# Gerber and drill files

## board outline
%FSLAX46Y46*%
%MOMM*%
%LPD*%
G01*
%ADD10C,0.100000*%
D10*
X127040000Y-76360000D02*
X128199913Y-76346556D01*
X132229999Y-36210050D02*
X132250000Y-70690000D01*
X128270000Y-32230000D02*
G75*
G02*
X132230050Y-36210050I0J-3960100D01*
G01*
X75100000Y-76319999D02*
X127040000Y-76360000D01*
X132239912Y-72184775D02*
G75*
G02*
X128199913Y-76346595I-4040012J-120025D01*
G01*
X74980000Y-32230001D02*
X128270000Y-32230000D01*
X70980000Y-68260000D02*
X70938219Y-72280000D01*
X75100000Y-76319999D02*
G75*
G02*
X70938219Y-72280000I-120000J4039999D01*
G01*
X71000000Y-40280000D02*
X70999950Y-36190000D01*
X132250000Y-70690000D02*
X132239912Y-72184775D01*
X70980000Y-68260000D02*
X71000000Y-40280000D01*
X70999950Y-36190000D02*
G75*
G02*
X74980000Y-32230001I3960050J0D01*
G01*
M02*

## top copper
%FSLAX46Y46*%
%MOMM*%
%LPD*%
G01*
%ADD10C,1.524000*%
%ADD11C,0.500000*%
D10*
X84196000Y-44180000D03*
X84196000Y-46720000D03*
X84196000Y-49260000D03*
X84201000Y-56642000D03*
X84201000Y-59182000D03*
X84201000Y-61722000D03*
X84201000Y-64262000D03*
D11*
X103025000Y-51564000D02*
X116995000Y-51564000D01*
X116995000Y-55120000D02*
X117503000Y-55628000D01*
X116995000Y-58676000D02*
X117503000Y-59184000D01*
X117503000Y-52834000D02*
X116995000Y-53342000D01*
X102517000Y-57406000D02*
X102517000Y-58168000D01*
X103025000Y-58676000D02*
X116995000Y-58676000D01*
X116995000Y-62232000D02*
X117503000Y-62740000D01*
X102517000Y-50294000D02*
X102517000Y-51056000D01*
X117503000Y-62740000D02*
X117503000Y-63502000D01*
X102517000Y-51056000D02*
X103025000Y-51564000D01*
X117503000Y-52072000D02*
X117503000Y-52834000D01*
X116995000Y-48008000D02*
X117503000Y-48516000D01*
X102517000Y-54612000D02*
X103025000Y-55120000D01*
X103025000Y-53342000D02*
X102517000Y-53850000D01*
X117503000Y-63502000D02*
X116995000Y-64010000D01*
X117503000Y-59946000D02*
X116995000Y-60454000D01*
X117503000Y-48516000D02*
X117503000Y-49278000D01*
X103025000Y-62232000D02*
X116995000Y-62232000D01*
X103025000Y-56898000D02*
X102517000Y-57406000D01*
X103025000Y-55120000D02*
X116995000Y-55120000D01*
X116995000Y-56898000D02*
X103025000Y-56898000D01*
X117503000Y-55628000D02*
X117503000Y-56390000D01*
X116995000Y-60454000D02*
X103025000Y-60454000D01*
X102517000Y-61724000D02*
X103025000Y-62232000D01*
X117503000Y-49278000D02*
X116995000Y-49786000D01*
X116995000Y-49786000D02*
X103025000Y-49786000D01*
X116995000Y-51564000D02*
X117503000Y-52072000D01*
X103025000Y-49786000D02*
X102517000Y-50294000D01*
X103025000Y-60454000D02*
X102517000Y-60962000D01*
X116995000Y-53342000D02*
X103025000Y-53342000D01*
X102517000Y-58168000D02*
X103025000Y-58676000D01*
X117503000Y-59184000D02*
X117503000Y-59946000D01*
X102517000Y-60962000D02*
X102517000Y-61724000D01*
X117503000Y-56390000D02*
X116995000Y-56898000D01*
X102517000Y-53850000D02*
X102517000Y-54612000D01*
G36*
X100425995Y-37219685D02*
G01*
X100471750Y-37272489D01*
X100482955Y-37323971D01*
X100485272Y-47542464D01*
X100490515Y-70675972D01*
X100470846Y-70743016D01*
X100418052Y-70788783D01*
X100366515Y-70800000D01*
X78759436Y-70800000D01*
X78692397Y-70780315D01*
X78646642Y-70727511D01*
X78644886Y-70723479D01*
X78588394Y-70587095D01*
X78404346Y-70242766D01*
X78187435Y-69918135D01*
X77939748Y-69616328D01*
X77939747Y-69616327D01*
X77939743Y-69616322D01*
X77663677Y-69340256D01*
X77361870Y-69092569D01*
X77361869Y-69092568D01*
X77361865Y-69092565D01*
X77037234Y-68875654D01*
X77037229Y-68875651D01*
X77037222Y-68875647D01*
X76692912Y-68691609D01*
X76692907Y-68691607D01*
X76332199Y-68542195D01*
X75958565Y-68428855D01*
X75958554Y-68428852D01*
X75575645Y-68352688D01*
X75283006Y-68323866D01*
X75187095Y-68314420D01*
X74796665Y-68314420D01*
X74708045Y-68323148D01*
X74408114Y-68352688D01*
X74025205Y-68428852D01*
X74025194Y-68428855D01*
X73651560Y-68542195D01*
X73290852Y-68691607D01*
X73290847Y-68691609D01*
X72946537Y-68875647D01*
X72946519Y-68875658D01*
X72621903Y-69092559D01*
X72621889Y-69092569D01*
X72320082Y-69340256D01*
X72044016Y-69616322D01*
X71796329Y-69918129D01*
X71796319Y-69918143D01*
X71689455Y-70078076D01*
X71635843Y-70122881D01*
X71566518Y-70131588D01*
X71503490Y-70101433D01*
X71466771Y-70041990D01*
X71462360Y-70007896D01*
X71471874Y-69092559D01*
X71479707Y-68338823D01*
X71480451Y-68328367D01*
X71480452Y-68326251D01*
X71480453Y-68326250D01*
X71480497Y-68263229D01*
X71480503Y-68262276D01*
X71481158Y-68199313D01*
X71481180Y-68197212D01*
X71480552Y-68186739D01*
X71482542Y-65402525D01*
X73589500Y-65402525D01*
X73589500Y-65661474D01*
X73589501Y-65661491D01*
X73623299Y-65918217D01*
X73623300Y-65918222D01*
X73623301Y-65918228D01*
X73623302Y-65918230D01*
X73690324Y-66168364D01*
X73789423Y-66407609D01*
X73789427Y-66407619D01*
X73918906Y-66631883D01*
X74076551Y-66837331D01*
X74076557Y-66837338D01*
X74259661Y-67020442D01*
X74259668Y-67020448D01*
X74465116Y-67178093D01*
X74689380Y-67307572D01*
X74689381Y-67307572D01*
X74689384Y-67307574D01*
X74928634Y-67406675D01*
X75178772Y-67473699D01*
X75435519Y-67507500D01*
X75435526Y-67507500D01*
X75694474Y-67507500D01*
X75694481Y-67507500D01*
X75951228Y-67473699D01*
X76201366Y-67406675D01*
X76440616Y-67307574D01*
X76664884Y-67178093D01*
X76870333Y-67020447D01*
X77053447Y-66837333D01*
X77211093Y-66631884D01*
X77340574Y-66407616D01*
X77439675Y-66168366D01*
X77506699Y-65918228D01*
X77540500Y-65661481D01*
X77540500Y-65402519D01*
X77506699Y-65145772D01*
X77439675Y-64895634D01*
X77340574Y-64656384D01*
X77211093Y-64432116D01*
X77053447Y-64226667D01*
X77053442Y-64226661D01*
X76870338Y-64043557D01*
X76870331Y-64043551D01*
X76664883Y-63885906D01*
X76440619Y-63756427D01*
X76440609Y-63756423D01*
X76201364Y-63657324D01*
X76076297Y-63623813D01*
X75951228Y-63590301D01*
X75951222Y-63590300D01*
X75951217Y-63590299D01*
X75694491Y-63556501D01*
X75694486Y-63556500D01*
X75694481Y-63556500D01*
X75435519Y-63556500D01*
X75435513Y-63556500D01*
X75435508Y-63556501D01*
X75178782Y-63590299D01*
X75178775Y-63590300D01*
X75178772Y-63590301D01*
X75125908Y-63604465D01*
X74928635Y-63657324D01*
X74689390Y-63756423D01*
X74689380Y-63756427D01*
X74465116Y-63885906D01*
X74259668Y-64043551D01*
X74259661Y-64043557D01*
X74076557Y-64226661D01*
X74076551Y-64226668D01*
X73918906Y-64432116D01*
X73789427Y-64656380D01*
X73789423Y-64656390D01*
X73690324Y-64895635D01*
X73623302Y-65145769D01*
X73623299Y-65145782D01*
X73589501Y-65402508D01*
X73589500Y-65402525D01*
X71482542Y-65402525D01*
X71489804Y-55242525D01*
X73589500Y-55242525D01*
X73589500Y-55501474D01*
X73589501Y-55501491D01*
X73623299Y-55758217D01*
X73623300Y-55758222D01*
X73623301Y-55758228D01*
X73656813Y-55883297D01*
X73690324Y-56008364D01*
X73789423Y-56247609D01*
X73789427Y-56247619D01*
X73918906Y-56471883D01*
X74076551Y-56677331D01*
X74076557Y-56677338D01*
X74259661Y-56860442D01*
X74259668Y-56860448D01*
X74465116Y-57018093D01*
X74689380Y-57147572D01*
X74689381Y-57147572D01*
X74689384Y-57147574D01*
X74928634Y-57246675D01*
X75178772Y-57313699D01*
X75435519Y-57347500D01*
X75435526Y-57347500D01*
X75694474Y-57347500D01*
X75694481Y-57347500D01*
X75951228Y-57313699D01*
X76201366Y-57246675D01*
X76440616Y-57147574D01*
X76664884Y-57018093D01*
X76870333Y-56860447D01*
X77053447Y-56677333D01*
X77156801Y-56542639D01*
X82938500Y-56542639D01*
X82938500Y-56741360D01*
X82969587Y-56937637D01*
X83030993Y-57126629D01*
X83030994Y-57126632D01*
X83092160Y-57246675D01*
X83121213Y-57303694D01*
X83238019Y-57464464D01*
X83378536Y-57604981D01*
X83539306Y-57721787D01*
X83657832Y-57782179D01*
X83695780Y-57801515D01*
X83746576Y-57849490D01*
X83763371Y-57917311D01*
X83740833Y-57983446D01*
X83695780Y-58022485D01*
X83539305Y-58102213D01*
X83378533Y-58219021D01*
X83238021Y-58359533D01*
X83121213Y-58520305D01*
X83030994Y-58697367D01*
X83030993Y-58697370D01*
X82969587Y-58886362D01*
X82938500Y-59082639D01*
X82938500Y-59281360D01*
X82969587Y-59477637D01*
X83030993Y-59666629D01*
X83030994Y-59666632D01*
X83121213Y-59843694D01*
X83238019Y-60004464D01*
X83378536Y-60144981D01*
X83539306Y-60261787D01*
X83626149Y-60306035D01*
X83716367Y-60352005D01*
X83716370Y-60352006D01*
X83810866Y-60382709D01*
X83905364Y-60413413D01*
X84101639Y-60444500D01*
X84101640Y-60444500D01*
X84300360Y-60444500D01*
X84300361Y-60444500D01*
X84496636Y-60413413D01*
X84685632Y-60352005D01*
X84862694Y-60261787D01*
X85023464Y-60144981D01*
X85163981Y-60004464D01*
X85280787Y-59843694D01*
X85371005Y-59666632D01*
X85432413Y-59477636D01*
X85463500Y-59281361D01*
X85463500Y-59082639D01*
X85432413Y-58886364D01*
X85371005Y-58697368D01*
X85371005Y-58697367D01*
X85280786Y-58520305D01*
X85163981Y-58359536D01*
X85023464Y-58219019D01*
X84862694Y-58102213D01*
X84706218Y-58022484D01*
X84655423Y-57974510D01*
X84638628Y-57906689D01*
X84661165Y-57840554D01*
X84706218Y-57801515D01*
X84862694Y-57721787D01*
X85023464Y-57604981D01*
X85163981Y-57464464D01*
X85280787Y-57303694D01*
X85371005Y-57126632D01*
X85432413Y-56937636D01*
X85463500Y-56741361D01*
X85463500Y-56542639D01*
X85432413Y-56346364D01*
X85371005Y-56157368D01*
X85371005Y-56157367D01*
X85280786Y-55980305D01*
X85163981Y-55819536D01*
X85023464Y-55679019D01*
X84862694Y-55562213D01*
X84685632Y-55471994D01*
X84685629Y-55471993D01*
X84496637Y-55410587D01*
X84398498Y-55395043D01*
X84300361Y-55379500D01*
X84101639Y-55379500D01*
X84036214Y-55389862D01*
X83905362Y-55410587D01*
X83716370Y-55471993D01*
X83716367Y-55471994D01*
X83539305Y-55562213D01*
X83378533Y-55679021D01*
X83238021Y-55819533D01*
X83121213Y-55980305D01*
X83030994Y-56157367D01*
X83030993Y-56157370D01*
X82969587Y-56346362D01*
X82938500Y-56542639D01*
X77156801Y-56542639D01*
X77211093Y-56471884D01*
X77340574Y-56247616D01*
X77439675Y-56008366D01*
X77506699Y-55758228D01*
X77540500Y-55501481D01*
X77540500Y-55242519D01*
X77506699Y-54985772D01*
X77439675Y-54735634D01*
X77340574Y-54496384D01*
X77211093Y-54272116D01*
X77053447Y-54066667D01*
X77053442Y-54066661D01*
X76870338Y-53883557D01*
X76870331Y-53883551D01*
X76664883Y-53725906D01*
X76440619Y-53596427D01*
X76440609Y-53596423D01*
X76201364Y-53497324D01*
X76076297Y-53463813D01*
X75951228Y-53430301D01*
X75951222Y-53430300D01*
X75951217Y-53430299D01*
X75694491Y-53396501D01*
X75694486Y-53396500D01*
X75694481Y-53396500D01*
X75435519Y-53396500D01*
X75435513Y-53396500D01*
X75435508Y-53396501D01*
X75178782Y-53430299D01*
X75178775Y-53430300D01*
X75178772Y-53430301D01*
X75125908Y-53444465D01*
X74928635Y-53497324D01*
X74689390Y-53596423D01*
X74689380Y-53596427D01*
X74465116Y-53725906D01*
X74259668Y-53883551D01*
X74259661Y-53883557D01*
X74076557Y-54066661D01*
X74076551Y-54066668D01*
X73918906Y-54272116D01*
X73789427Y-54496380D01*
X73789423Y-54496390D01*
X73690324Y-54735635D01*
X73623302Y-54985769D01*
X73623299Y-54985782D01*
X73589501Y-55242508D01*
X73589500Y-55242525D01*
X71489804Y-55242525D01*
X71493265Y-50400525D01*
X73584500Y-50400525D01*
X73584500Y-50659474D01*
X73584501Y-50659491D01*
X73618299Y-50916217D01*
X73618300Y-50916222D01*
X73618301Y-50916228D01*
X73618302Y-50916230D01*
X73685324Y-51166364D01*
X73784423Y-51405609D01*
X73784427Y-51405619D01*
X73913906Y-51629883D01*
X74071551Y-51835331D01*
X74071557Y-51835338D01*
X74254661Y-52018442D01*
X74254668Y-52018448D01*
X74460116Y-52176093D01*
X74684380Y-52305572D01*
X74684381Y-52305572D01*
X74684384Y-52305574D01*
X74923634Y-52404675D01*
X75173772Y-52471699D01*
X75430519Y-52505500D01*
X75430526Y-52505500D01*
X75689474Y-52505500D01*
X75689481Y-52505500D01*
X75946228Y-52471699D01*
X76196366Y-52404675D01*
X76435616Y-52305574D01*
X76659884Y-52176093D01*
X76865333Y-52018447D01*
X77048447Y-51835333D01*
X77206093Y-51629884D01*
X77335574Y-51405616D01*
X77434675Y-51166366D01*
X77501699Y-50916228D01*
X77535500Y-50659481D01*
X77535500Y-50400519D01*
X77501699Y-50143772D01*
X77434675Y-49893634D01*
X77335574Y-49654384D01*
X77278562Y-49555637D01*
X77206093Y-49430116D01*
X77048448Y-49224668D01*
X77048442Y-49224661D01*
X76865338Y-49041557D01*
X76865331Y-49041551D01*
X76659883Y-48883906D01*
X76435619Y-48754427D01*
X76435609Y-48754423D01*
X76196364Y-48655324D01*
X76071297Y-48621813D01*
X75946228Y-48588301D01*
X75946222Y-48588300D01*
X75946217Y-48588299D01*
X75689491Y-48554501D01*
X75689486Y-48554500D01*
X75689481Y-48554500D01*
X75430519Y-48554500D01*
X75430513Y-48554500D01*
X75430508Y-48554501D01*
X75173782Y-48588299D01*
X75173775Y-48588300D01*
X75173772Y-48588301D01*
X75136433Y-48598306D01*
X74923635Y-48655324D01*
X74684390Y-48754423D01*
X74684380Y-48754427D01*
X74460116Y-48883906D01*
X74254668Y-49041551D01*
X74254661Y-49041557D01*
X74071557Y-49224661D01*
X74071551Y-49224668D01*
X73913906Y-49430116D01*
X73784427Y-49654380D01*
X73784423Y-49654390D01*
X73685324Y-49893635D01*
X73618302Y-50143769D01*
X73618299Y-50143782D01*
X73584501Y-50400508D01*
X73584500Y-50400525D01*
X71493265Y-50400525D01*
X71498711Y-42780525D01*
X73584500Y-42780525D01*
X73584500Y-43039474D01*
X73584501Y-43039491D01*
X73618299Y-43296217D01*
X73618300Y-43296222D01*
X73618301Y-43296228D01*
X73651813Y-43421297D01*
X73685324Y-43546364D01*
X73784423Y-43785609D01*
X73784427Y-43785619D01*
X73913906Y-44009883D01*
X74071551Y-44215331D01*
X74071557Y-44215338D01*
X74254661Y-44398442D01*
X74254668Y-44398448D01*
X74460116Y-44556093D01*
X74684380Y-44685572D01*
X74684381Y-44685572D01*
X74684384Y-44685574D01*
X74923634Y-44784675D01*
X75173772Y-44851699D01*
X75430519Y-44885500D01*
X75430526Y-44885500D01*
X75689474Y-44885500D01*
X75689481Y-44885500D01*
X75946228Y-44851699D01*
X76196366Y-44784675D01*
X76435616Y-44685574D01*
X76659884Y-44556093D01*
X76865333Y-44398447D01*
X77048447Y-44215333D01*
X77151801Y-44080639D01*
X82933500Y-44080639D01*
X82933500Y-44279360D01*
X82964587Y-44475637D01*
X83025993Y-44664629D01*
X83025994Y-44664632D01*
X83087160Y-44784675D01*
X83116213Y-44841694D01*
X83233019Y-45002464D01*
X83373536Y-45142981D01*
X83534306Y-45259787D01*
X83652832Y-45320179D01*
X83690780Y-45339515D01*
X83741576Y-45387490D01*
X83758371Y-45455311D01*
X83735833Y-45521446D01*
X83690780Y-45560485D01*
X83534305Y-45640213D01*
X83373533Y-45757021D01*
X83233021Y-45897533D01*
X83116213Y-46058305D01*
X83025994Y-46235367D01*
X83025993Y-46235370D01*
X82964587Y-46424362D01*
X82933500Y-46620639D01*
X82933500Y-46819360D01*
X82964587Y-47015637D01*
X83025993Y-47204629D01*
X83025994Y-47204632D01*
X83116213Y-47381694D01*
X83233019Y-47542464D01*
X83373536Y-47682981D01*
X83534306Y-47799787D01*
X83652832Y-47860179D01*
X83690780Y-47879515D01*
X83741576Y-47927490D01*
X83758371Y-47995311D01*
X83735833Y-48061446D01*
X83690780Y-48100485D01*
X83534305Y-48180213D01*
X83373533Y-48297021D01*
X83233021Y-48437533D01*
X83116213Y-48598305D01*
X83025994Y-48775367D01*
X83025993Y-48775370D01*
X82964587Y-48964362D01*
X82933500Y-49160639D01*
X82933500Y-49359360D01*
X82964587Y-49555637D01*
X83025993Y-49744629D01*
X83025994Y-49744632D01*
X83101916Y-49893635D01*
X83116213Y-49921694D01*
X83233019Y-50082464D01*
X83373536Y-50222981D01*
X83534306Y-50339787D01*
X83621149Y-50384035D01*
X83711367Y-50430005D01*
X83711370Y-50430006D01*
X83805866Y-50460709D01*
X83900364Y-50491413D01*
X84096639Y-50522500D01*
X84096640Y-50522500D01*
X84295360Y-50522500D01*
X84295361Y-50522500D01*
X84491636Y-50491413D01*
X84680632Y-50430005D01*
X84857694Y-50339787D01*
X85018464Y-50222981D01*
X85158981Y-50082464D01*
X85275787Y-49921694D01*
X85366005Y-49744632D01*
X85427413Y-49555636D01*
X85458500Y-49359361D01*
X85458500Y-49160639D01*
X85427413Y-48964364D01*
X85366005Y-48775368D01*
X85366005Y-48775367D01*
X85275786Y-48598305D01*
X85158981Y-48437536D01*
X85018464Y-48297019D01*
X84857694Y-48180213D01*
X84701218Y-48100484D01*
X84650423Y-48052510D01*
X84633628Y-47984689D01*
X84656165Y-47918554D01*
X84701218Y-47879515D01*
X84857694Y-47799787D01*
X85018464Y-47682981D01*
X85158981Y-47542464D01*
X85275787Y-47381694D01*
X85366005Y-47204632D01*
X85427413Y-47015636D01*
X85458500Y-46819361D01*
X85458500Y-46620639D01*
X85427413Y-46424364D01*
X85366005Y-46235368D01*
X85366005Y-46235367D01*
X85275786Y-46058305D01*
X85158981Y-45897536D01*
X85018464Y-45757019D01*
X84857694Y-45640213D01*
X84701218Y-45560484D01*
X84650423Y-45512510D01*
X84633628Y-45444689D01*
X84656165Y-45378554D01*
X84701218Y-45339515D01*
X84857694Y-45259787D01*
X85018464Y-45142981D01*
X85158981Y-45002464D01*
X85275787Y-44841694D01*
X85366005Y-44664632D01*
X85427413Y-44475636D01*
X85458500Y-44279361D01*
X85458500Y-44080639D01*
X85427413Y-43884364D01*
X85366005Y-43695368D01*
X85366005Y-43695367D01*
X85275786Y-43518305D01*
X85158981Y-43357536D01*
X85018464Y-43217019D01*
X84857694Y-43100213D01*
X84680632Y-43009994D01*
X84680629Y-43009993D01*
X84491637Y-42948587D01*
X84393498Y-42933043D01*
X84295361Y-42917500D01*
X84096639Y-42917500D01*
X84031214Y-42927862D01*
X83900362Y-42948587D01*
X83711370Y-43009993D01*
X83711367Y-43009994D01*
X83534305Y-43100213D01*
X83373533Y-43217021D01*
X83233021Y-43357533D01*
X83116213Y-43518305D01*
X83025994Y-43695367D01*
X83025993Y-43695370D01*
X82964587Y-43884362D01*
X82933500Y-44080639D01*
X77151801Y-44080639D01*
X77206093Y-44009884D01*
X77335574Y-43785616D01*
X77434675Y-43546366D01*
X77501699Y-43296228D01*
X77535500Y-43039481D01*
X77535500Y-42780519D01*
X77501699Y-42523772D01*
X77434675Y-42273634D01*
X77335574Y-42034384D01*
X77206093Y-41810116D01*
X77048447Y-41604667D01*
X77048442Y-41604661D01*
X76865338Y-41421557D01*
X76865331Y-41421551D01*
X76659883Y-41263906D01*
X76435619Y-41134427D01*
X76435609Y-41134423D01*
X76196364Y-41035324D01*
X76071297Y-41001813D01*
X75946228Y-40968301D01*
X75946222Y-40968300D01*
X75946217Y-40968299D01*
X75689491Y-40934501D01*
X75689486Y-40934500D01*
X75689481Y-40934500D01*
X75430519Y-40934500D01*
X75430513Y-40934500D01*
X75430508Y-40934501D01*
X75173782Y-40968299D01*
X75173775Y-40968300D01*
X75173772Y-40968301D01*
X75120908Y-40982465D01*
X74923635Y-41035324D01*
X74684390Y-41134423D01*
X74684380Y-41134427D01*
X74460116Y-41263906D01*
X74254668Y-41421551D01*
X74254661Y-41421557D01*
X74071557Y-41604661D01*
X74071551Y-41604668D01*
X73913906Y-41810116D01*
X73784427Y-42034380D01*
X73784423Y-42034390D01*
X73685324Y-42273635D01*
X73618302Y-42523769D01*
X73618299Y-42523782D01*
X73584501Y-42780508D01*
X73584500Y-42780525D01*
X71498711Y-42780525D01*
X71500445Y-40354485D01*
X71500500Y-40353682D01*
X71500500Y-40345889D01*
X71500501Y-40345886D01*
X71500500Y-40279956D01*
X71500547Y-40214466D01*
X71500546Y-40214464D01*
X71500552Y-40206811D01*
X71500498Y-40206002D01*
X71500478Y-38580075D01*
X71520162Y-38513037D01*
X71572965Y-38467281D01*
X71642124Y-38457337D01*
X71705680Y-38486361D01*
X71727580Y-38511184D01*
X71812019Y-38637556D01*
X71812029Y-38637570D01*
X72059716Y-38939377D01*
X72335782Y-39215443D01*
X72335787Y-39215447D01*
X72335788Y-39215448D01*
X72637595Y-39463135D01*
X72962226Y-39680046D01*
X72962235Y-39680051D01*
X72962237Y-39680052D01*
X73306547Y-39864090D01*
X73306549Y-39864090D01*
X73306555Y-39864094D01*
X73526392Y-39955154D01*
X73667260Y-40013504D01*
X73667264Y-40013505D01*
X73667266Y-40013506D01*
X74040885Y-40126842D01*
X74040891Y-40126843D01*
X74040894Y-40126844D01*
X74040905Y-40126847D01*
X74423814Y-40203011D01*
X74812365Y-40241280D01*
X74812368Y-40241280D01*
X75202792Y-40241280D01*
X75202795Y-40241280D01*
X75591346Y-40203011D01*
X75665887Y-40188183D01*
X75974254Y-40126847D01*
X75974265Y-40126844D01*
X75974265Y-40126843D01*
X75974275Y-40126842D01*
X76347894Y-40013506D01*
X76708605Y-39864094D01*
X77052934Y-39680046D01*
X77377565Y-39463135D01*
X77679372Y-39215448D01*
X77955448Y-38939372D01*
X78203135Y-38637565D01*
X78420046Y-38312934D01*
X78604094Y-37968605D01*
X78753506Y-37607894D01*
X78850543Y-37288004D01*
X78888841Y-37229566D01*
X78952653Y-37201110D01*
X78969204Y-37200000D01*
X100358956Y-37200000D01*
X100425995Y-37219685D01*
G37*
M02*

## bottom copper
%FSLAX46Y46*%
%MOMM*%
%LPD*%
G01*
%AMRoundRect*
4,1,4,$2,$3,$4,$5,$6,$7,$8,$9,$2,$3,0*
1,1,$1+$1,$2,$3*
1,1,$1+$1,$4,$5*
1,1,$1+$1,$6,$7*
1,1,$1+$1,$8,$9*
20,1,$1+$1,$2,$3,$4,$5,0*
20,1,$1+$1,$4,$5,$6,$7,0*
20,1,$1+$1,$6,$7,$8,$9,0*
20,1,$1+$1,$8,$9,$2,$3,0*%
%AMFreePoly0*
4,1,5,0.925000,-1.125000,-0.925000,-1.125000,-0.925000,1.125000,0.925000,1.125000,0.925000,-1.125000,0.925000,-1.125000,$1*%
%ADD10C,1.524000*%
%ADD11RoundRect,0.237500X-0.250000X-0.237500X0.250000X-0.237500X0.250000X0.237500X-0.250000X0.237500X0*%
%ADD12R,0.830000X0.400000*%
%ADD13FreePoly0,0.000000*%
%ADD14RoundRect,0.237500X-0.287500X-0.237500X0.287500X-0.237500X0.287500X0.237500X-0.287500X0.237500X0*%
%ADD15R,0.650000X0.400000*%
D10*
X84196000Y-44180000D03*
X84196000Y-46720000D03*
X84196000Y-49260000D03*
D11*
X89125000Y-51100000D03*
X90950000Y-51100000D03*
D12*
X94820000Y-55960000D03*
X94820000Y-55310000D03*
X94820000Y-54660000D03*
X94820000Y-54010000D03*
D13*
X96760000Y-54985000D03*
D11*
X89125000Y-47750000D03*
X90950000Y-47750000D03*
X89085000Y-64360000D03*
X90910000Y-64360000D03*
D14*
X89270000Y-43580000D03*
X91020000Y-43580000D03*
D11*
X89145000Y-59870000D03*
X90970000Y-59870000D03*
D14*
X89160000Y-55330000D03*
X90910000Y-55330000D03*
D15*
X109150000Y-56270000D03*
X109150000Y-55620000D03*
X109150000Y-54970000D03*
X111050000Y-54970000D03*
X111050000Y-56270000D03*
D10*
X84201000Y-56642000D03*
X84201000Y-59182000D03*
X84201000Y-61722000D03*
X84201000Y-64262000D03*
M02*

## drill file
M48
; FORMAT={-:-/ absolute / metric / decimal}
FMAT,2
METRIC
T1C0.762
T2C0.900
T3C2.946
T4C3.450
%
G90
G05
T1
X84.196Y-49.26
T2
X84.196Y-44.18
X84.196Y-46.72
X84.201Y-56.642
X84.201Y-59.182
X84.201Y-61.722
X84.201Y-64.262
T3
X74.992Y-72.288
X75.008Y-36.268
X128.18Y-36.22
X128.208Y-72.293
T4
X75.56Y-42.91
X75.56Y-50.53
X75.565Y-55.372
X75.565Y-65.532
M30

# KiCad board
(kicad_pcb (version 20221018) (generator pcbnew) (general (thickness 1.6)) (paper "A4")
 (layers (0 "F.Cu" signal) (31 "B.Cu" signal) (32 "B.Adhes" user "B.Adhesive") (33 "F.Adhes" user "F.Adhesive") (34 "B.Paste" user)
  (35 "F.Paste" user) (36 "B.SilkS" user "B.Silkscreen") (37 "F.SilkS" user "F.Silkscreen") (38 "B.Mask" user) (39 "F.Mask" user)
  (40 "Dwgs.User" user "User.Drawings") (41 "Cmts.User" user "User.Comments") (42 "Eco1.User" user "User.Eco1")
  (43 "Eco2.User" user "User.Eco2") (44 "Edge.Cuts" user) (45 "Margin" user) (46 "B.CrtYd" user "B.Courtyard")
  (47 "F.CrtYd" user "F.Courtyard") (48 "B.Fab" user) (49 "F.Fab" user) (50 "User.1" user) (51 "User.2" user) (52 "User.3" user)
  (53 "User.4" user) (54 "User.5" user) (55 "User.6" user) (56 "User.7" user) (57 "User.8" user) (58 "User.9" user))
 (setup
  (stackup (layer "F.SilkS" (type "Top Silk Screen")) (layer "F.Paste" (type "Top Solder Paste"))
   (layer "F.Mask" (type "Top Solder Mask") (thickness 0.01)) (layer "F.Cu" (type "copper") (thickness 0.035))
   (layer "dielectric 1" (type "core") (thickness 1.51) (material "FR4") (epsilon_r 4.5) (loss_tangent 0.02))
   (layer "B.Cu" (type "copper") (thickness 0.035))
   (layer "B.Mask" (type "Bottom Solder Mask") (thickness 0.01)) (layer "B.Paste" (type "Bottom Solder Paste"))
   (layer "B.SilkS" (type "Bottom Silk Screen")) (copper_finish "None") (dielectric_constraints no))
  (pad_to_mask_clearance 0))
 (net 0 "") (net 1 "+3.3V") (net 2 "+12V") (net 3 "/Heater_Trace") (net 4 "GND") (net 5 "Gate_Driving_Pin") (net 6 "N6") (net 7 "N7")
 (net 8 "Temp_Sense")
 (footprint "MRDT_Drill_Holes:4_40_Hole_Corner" (layer "F.Cu") (at 79 68.28 180)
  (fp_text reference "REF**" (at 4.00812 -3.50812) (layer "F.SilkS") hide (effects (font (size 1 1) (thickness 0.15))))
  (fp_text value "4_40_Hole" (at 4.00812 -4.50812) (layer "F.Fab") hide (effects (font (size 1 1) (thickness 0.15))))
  (pad "" np_thru_hole circle (at 4.00812 -4.00812 180) (size 2.9464 2.9464) (drill 2.9464) (layers "*.Cu" "*.Mask") (clearance 2.5)))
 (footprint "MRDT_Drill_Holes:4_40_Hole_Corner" (layer "F.Cu") (at 79.0157 40.2757 90)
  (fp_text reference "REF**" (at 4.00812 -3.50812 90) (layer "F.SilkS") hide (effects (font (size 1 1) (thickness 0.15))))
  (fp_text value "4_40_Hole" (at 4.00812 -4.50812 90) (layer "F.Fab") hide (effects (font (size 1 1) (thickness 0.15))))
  (pad "" np_thru_hole circle (at 4.00812 -4.00812 90) (size 2.9464 2.9464) (drill 2.9464) (layers "*.Cu" "*.Mask") (clearance 2.5)))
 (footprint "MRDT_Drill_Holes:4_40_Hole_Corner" (layer "F.Cu") (at 124.199913 68.284775 -90)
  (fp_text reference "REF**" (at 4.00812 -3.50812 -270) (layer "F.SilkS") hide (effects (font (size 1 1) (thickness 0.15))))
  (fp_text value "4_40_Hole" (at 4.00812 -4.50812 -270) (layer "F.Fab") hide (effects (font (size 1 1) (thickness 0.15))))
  (pad "" np_thru_hole circle (at 4.00812 -4.00812 270) (size 2.9464 2.9464) (drill 2.9464) (layers "*.Cu" "*.Mask") (clearance 2.5)))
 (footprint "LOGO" (layer "F.Cu") (at 96.09 65.32)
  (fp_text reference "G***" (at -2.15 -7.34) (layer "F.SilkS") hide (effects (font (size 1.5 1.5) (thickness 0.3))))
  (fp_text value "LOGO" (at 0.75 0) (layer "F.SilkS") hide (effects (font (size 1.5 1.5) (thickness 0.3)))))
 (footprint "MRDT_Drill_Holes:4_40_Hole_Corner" (layer "F.Cu") (at 124.171879 40.22817)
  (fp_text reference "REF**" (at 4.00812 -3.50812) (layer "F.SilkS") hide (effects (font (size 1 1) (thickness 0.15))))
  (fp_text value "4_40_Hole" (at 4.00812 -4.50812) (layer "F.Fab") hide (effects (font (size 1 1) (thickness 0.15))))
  (pad "" np_thru_hole circle (at 4.00812 -4.00812) (size 2.9464 2.9464) (drill 2.9464) (layers "*.Cu" "*.Mask") (clearance 2.5)))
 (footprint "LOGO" (layer "F.Cu") (at 111.506 50.8)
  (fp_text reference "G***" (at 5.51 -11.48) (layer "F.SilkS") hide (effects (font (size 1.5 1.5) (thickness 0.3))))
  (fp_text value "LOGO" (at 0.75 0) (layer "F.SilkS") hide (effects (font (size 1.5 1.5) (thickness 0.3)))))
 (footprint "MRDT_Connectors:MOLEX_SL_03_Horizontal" (layer "B.Cu") (at 84.196 44.18 -90)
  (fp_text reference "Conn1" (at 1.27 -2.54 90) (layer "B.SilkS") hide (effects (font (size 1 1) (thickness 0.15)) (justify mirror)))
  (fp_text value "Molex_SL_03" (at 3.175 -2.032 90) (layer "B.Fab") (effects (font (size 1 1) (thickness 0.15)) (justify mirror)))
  (pad "" np_thru_hole circle (at -1.27 8.636 270) (size 3.45 3.45) (drill 3.45) (layers "*.Cu" "*.Mask"))
  (pad "" np_thru_hole circle (at 6.35 8.636 270) (size 3.45 3.45) (drill 3.45) (layers "*.Cu" "*.Mask"))
  (pad "1" thru_hole circle (at 0 0 270) (size 1.524 1.524) (drill 0.9) (layers "*.Cu" "*.Mask") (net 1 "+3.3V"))
  (pad "2" thru_hole circle (at 2.54 0 270) (size 1.524 1.524) (drill 0.9) (layers "*.Cu" "*.Mask") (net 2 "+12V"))
  (pad "3" thru_hole circle (at 5.08 0 270) (size 1.524 1.524) (drill 0.762) (layers "*.Cu" "*.Mask") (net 2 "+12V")))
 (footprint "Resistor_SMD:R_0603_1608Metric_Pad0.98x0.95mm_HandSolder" (layer "B.Cu") (at 90.0375 51.1)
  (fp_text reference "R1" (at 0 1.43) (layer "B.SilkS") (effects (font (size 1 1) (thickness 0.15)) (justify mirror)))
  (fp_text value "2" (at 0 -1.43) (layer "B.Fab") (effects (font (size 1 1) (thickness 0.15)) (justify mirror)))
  (pad "1" smd roundrect (at -0.9125 0) (size 0.975 0.95) (layers "B.Cu" "B.Paste" "B.Mask") (roundrect_rratio 0.25) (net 2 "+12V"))
  (pad "2" smd roundrect (at 0.9125 0) (size 0.975 0.95) (layers "B.Cu" "B.Paste" "B.Mask") (roundrect_rratio 0.25) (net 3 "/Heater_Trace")))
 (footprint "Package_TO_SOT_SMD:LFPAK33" (layer "B.Cu") (at 96.355 54.985) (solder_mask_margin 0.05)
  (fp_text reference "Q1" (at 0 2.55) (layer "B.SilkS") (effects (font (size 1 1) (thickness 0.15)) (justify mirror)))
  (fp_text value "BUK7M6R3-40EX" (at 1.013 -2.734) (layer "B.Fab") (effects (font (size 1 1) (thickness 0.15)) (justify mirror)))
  (pad "" smd rect (at -1.535 -0.975) (size 0.83 0.3) (layers "B.Paste"))
  (pad "" smd rect (at -1.535 -0.325) (size 0.83 0.3) (layers "B.Paste"))
  (pad "" smd rect (at -1.535 0.325) (size 0.83 0.3) (layers "B.Paste"))
  (pad "" smd rect (at -1.535 0.975) (size 0.83 0.3) (layers "B.Paste"))
  (pad "" smd rect (at -0.215 -0.626) (size 0.51 0.635) (layers "B.Paste"))
  (pad "" smd rect (at -0.215 0.626) (size 0.51 0.635) (layers "B.Paste"))
  (pad "" smd rect (at 0.645 -0.626) (size 0.51 0.635) (layers "B.Paste"))
  (pad "" smd rect (at 0.645 0.626) (size 0.51 0.635) (layers "B.Paste"))
  (pad "" smd rect (at 1.575 -0.975) (size 0.75 0.3) (layers "B.Paste"))
  (pad "" smd rect (at 1.575 -0.325) (size 0.75 0.3) (layers "B.Paste"))
  (pad "" smd rect (at 1.575 0.325) (size 0.75 0.3) (layers "B.Paste"))
  (pad "" smd rect (at 1.575 0.975) (size 0.75 0.3) (layers "B.Paste"))
  (pad "1" smd rect (at -1.535 0.975) (size 0.83 0.4) (layers "B.Cu" "B.Mask") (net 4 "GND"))
  (pad "2" smd rect (at -1.535 0.325) (size 0.83 0.4) (layers "B.Cu" "B.Mask") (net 4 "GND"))
  (pad "3" smd rect (at -1.535 -0.325) (size 0.83 0.4) (layers "B.Cu" "B.Mask") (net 4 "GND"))
  (pad "4" smd rect (at -1.535 -0.975) (size 0.83 0.4) (layers "B.Cu" "B.Mask") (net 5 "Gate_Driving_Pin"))
  (pad "5" smd custom (at 0.405 0) (size 1.85 2.25) (layers "B.Cu" "B.Mask") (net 3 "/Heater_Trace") (zone_connect 2)
   (thermal_bridge_angle 45) (options (clearance outline) (anchor rect)) (primitives)))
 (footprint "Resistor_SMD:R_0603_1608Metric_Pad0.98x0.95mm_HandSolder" (layer "B.Cu") (at 90.0375 47.75)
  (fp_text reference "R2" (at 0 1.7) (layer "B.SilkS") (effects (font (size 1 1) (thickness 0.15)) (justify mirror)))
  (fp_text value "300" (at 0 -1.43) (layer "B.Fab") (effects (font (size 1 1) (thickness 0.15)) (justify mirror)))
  (pad "1" smd roundrect (at -0.9125 0) (size 0.975 0.95) (layers "B.Cu" "B.Paste" "B.Mask") (roundrect_rratio 0.25) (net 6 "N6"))
  (pad "2" smd roundrect (at 0.9125 0) (size 0.975 0.95) (layers "B.Cu" "B.Paste" "B.Mask") (roundrect_rratio 0.25) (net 4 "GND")))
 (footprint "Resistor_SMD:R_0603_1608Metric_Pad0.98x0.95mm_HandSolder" (layer "B.Cu") (at 89.9975 64.36)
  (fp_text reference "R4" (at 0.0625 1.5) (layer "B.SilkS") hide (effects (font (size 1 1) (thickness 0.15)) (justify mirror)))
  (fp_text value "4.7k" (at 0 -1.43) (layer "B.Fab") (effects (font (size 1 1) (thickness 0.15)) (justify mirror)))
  (pad "1" smd roundrect (at -0.9125 0) (size 0.975 0.95) (layers "B.Cu" "B.Paste" "B.Mask") (roundrect_rratio 0.25)
   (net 5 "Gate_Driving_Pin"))
  (pad "2" smd roundrect (at 0.9125 0) (size 0.975 0.95) (layers "B.Cu" "B.Paste" "B.Mask") (roundrect_rratio 0.25) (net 4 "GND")))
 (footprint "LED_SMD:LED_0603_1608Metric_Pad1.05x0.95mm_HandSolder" (layer "B.Cu") (at 90.145 43.58)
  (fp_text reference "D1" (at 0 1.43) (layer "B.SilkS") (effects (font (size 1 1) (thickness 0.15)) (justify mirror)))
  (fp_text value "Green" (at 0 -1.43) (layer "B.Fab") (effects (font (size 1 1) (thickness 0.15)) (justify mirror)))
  (pad "1" smd roundrect (at -0.875 0) (size 1.05 0.95) (layers "B.Cu" "B.Paste" "B.Mask") (roundrect_rratio 0.25) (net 6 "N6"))
  (pad "2" smd roundrect (at 0.875 0) (size 1.05 0.95) (layers "B.Cu" "B.Paste" "B.Mask") (roundrect_rratio 0.25) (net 1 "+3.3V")))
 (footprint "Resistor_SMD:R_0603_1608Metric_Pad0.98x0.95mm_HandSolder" (layer "B.Cu") (at 90.0575 59.87)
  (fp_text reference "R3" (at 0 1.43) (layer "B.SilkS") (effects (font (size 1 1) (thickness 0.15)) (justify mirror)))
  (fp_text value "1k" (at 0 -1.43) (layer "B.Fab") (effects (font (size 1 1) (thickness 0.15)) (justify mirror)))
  (pad "1" smd roundrect (at -0.9125 0) (size 0.975 0.95) (layers "B.Cu" "B.Paste" "B.Mask") (roundrect_rratio 0.25) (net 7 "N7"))
  (pad "2" smd roundrect (at 0.9125 0) (size 0.975 0.95) (layers "B.Cu" "B.Paste" "B.Mask") (roundrect_rratio 0.25) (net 4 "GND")))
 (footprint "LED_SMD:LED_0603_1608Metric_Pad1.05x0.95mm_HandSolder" (layer "B.Cu") (at 90.035 55.33)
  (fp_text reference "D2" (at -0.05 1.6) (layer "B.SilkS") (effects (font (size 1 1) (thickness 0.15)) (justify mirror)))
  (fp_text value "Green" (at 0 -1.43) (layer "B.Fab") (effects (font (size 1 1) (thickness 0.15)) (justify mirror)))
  (pad "1" smd roundrect (at -0.875 0) (size 1.05 0.95) (layers "B.Cu" "B.Paste" "B.Mask") (roundrect_rratio 0.25) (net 7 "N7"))
  (pad "2" smd roundrect (at 0.875 0) (size 1.05 0.95) (layers "B.Cu" "B.Paste" "B.Mask") (roundrect_rratio 0.25) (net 2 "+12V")))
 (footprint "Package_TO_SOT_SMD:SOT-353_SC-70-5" (layer "B.Cu") (at 110.1 55.62)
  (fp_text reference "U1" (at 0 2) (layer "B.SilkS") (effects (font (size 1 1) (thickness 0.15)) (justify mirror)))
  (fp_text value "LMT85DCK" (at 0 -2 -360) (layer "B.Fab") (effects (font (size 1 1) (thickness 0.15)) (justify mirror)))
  (pad "1" smd rect (at -0.95 0.65) (size 0.65 0.4) (layers "B.Cu" "B.Paste" "B.Mask") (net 1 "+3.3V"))
  (pad "2" smd rect (at -0.95 0) (size 0.65 0.4) (layers "B.Cu" "B.Paste" "B.Mask") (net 4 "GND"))
  (pad "3" smd rect (at -0.95 -0.65) (size 0.65 0.4) (layers "B.Cu" "B.Paste" "B.Mask") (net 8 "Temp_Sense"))
  (pad "4" smd rect (at 0.95 -0.65) (size 0.65 0.4) (layers "B.Cu" "B.Paste" "B.Mask") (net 1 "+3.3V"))
  (pad "5" smd rect (at 0.95 0.65) (size 0.65 0.4) (layers "B.Cu" "B.Paste" "B.Mask") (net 4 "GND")))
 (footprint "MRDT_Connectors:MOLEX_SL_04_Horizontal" (layer "B.Cu") (at 84.201 56.642 -90)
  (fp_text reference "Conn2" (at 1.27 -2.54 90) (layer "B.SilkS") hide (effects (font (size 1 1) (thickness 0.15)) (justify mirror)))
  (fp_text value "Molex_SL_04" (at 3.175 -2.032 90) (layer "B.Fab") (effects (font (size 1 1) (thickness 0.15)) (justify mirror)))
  (pad "" np_thru_hole circle (at -1.27 8.636 270) (size 3.45 3.45) (drill 3.45) (layers "*.Cu" "*.Mask"))
  (pad "" np_thru_hole circle (at 8.89 8.636 270) (size 3.45 3.45) (drill 3.45) (layers "*.Cu" "*.Mask"))
  (pad "1" thru_hole circle (at 0 0 270) (size 1.524 1.524) (drill 0.9) (layers "*.Cu" "*.Mask") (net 5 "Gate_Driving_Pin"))
  (pad "2" thru_hole circle (at 2.54 0 270) (size 1.524 1.524) (drill 0.9) (layers "*.Cu" "*.Mask") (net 8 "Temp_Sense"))
  (pad "3" thru_hole circle (at 5.08 0 270) (size 1.524 1.524) (drill 0.9) (layers "*.Cu" "*.Mask") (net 4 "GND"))
  (pad "4" thru_hole circle (at 7.62 0 270) (size 1.524 1.524) (drill 0.9) (layers "*.Cu" "*.Mask") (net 4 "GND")))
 (gr_line (start 127.04 76.36) (end 128.199913 76.346556) (stroke (width 0.1) (type default)) (layer "Edge.Cuts"))
 (gr_line (start 132.229999 36.21005) (end 132.25 70.69) (stroke (width 0.1) (type default)) (layer "Edge.Cuts"))
 (gr_arc (start 128.27 32.23) (mid 131.07724 33.396952) (end 132.229999 36.21005) (stroke (width 0.1) (type default)) (layer "Edge.Cuts"))
 (gr_line (start 75.1 76.319999) (end 127.04 76.36) (stroke (width 0.1) (type default)) (layer "Edge.Cuts"))
 (gr_arc (start 132.239912 72.184775) (mid 131.1 75.12) (end 128.199913 76.346556) (stroke (width 0.1) (type default)) (layer "Edge.Cuts"))
 (gr_line (start 74.98 32.230001) (end 128.27 32.23) (stroke (width 0.1) (type default)) (layer "Edge.Cuts"))
 (gr_line (start 70.98 68.26) (end 70.938219 72.28) (stroke (width 0.1) (type default)) (layer "Edge.Cuts"))
 (gr_arc (start 75.1 76.319999) (mid 72.164775 75.180087) (end 70.938219 72.28) (stroke (width 0.1) (type default)) (layer "Edge.Cuts"))
 (gr_line (start 71 40.28) (end 70.99995 36.19) (stroke (width 0.1) (type default)) (layer "Edge.Cuts"))
 (gr_line (start 132.25 70.69) (end 132.239912 72.184775) (stroke (width 0.1) (type default)) (layer "Edge.Cuts"))
 (gr_line (start 70.98 68.26) (end 71 40.28) (stroke (width 0.1) (type default)) (layer "Edge.Cuts"))
 (gr_arc (start 70.99995 36.19) (mid 72.166902 33.38276) (end 74.98 32.230001) (stroke (width 0.1) (type default)) (layer "Edge.Cuts"))
 (segment (start 103.025 51.564) (end 116.995 51.564) (width 0.5) (layer "F.Cu") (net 3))
 (segment (start 116.995 55.12) (end 117.503 55.628) (width 0.5) (layer "F.Cu") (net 3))
 (segment (start 116.995 58.676) (end 117.503 59.184) (width 0.5) (layer "F.Cu") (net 3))
 (segment (start 117.503 52.834) (end 116.995 53.342) (width 0.5) (layer "F.Cu") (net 3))
 (segment (start 102.517 57.406) (end 102.517 58.168) (width 0.5) (layer "F.Cu") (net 3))
 (segment (start 103.025 58.676) (end 116.995 58.676) (width 0.5) (layer "F.Cu") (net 3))
 (segment (start 116.995 62.232) (end 117.503 62.74) (width 0.5) (layer "F.Cu") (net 3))
 (segment (start 102.517 50.294) (end 102.517 51.056) (width 0.5) (layer "F.Cu") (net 3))
 (segment (start 117.503 62.74) (end 117.503 63.502) (width 0.5) (layer "F.Cu") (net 3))
 (segment (start 102.517 51.056) (end 103.025 51.564) (width 0.5) (layer "F.Cu") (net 3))
 (segment (start 117.503 52.072) (end 117.503 52.834) (width 0.5) (layer "F.Cu") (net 3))
 (segment (start 116.995 48.008) (end 117.503 48.516) (width 0.5) (layer "F.Cu") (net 3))
 (segment (start 102.517 54.612) (end 103.025 55.12) (width 0.5) (layer "F.Cu") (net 3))
 (segment (start 103.025 53.342) (end 102.517 53.85) (width 0.5) (layer "F.Cu") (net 3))
 (segment (start 117.503 63.502) (end 116.995 64.01) (width 0.5) (layer "F.Cu") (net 3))
 (segment (start 117.503 59.946) (end 116.995 60.454) (width 0.5) (layer "F.Cu") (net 3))
 (segment (start 117.503 48.516) (end 117.503 49.278) (width 0.5) (layer "F.Cu") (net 3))
 (segment (start 103.025 62.232) (end 116.995 62.232) (width 0.5) (layer "F.Cu") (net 3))
 (segment (start 103.025 56.898) (end 102.517 57.406) (width 0.5) (layer "F.Cu") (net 3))
 (segment (start 103.025 55.12) (end 116.995 55.12) (width 0.5) (layer "F.Cu") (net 3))
 (segment (start 116.995 56.898) (end 103.025 56.898) (width 0.5) (layer "F.Cu") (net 3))
 (segment (start 117.503 55.628) (end 117.503 56.39) (width 0.5) (layer "F.Cu") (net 3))
 (segment (start 116.995 60.454) (end 103.025 60.454) (width 0.5) (layer "F.Cu") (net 3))
 (segment (start 102.517 61.724) (end 103.025 62.232) (width 0.5) (layer "F.Cu") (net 3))
 (segment (start 117.503 49.278) (end 116.995 49.786) (width 0.5) (layer "F.Cu") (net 3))
 (segment (start 116.995 49.786) (end 103.025 49.786) (width 0.5) (layer "F.Cu") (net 3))
 (segment (start 116.995 51.564) (end 117.503 52.072) (width 0.5) (layer "F.Cu") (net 3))
 (segment (start 103.025 49.786) (end 102.517 50.294) (width 0.5) (layer "F.Cu") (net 3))
 (segment (start 103.025 60.454) (end 102.517 60.962) (width 0.5) (layer "F.Cu") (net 3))
 (segment (start 116.995 53.342) (end 103.025 53.342) (width 0.5) (layer "F.Cu") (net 3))
 (segment (start 102.517 58.168) (end 103.025 58.676) (width 0.5) (layer "F.Cu") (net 3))
 (segment (start 117.503 59.184) (end 117.503 59.946) (width 0.5) (layer "F.Cu") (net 3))
 (segment (start 102.517 60.962) (end 102.517 61.724) (width 0.5) (layer "F.Cu") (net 3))
 (segment (start 117.503 56.39) (end 116.995 56.898) (width 0.5) (layer "F.Cu") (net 3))
 (segment (start 102.517 53.85) (end 102.517 54.612) (width 0.5) (layer "F.Cu") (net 3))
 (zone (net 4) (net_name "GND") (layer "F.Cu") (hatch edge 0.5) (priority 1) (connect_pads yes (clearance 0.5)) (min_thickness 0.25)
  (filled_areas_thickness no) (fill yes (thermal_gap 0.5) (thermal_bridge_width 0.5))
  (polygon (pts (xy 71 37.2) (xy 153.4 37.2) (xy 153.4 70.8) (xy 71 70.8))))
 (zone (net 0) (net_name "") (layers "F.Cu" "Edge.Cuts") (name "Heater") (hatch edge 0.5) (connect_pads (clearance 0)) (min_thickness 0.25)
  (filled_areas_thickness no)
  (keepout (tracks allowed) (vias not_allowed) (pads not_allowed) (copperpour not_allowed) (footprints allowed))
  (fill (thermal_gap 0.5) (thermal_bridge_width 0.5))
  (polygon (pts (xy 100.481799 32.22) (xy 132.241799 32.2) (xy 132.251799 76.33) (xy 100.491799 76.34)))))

